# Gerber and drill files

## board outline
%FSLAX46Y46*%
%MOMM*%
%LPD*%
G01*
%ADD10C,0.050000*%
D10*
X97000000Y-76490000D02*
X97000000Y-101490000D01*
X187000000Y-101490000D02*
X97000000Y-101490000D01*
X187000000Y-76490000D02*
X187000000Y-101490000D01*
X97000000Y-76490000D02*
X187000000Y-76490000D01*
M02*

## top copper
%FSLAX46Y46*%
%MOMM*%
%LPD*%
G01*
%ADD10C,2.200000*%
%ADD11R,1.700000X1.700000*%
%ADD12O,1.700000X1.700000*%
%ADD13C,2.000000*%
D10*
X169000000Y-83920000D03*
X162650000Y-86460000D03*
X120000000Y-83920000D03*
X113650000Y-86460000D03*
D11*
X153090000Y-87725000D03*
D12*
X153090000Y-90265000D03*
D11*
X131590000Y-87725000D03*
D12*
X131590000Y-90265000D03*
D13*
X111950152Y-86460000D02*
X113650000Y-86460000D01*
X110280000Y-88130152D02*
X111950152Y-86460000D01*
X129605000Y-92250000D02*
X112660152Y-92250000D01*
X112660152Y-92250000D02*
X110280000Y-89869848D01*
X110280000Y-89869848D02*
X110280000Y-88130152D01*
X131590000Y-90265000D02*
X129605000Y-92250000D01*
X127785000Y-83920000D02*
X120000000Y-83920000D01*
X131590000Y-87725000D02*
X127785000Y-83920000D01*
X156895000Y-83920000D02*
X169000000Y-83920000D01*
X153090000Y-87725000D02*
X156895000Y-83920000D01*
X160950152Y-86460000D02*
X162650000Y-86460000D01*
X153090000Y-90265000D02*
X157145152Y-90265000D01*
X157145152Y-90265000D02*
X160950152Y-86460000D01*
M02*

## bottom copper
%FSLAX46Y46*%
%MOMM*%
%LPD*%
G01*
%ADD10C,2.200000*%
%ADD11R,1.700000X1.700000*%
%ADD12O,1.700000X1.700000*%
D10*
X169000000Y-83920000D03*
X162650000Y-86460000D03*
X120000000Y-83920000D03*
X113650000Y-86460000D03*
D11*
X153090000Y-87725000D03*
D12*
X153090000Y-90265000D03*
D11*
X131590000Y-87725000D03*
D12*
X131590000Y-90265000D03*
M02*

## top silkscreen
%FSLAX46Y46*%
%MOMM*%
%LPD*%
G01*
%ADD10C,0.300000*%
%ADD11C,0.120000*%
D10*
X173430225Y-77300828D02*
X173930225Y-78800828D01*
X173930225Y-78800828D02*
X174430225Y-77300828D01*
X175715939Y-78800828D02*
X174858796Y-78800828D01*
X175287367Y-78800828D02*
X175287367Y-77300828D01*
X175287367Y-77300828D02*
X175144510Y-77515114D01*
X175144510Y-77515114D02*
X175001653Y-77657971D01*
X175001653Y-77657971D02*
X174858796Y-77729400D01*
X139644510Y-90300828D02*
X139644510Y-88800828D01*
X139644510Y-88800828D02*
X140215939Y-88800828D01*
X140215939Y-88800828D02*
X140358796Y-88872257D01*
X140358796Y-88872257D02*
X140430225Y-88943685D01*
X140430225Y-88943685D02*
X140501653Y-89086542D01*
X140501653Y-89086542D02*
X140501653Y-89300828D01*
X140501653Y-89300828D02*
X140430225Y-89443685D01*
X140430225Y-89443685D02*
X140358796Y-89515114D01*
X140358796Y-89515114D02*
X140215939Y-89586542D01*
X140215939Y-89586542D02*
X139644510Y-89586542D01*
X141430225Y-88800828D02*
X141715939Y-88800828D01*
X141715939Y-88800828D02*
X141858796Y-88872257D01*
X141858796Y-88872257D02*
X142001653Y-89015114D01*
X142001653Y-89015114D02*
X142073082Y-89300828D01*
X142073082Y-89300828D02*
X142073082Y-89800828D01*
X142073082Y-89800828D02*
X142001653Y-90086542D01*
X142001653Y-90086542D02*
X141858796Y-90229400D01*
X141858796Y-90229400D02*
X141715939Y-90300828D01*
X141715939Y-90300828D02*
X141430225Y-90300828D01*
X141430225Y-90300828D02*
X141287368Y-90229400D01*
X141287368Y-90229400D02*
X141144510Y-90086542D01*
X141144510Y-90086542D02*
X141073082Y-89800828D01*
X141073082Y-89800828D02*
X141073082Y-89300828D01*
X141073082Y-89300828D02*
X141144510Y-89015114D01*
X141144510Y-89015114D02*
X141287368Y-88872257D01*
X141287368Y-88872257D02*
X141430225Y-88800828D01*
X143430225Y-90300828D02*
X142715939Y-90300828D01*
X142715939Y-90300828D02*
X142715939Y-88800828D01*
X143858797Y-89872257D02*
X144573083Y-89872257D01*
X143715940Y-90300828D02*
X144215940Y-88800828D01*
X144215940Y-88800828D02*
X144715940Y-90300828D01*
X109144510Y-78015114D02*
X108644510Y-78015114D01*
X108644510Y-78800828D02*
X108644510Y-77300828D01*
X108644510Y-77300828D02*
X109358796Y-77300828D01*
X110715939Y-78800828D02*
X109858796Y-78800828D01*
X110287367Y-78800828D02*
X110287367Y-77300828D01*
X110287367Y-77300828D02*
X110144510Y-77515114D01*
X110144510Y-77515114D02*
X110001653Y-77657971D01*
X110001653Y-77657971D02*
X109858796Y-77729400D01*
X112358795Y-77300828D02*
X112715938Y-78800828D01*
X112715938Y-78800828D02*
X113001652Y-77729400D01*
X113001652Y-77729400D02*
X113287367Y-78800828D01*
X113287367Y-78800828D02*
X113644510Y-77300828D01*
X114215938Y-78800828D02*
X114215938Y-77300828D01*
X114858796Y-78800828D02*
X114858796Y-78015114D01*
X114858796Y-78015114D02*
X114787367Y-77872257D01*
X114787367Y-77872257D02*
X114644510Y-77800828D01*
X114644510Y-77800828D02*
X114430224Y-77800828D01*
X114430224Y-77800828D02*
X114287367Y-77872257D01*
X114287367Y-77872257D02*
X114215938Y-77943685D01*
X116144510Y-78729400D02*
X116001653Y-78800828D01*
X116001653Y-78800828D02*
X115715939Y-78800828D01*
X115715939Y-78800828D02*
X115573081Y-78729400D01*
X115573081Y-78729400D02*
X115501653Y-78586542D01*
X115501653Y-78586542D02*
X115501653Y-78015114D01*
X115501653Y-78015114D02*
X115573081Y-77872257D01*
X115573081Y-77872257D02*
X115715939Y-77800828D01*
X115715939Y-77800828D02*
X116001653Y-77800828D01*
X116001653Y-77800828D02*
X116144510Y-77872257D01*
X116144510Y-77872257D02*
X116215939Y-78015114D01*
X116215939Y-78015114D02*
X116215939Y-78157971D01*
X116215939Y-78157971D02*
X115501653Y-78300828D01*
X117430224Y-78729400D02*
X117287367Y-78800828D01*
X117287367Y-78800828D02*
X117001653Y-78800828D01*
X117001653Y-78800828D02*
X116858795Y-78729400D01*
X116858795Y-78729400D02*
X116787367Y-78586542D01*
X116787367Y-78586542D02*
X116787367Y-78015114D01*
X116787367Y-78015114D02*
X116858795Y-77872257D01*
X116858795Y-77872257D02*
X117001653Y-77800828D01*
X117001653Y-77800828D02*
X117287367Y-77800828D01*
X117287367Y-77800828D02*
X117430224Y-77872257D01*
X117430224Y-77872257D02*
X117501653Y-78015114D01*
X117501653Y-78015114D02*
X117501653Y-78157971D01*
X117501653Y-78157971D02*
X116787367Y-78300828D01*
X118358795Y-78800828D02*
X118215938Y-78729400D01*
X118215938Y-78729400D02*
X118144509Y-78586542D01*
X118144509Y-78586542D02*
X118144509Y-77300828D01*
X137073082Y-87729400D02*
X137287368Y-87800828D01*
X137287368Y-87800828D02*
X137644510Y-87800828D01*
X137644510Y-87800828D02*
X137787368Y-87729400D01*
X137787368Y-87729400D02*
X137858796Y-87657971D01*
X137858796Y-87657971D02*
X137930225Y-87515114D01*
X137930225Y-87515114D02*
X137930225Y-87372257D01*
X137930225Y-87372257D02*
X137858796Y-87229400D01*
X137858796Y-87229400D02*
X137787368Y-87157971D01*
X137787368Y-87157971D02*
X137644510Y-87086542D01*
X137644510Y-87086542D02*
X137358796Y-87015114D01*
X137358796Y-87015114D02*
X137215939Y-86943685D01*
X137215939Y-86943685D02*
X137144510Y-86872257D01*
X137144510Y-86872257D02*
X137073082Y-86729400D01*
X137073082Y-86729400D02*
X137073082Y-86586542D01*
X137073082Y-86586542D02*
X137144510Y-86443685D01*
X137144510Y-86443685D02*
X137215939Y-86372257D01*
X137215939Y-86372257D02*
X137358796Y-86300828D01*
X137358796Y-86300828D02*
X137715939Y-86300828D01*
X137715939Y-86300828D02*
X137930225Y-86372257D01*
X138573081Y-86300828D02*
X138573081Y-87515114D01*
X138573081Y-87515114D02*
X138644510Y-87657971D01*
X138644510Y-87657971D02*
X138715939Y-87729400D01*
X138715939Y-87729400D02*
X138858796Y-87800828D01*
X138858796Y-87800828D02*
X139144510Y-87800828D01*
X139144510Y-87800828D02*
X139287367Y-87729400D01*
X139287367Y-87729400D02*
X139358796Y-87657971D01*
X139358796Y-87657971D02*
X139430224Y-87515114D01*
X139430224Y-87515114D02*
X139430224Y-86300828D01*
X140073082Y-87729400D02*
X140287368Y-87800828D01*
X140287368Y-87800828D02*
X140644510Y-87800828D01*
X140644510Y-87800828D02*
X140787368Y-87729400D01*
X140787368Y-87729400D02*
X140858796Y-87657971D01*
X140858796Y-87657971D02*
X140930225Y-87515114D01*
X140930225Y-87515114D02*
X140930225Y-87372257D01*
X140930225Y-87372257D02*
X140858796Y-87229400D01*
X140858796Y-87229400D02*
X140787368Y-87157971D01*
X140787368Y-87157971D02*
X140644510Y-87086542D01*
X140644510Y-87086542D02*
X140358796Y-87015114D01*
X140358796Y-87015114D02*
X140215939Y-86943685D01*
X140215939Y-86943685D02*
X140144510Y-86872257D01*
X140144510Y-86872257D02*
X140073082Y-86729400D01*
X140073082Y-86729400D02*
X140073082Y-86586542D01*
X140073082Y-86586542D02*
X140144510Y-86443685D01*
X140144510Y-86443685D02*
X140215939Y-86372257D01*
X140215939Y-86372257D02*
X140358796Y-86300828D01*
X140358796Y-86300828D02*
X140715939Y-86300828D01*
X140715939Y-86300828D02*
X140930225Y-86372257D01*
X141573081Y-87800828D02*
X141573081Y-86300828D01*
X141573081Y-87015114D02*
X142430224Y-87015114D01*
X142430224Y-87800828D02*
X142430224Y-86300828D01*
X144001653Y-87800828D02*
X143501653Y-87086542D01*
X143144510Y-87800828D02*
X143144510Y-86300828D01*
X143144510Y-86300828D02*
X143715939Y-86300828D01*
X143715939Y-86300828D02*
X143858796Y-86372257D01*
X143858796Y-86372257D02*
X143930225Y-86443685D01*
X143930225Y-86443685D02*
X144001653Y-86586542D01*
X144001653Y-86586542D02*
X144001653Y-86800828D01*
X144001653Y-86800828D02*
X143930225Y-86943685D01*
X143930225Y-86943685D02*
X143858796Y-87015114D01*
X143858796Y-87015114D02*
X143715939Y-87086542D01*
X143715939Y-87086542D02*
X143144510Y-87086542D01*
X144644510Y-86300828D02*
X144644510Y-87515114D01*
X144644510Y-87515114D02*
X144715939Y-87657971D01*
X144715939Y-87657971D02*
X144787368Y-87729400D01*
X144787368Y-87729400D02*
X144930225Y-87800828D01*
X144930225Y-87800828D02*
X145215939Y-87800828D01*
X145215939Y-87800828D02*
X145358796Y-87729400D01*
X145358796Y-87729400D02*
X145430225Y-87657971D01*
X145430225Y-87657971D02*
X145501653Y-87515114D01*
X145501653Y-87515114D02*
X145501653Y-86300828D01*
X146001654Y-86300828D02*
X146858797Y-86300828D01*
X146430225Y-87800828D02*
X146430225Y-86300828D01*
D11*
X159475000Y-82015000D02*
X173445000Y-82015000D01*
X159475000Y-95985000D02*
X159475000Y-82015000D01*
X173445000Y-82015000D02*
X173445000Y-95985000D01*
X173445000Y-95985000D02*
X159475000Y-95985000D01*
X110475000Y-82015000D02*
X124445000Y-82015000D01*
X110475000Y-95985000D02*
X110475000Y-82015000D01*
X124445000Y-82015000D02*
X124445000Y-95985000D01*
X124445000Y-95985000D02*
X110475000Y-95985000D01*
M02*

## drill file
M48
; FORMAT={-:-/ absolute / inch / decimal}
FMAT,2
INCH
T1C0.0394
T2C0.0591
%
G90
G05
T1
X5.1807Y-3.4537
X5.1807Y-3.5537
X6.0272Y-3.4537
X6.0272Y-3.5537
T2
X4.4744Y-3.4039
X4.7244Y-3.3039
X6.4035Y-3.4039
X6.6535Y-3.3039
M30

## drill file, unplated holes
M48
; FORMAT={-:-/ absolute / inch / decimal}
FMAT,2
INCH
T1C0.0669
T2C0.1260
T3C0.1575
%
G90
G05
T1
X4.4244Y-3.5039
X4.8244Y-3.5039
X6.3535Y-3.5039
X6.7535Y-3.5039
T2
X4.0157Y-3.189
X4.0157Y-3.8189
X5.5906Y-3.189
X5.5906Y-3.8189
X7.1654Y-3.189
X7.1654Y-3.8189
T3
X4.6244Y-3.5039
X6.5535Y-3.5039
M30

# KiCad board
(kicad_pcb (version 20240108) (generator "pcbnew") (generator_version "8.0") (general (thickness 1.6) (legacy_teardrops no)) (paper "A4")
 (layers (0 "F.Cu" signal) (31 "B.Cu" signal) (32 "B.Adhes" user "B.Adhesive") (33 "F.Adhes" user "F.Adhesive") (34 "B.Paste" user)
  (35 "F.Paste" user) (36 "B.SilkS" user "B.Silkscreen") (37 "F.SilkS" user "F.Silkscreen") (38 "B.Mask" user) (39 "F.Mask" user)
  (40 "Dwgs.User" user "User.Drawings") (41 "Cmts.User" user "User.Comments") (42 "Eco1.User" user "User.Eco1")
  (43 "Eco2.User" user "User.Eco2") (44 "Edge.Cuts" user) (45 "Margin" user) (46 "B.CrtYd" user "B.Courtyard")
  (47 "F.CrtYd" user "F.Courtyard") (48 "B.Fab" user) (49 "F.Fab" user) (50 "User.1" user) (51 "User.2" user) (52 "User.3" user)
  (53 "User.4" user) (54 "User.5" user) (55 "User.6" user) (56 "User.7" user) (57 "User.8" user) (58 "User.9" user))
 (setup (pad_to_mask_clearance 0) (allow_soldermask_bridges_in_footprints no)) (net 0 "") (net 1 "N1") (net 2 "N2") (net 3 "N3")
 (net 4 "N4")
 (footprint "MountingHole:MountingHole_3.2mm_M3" (layer "F.Cu") (at 142 81)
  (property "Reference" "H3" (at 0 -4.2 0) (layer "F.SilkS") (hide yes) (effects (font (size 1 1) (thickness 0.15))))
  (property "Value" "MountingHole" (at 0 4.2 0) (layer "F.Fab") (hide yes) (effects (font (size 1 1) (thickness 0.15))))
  (pad "" np_thru_hole circle (at 0 0) (size 3.2 3.2) (drill 3.2) (layers "*.Cu" "*.Mask")))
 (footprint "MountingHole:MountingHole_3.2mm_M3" (layer "F.Cu") (at 142 97)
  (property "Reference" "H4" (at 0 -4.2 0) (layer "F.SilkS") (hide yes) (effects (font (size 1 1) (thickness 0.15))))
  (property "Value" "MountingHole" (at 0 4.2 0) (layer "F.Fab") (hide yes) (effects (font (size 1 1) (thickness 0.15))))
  (pad "" np_thru_hole circle (at 0 0) (size 3.2 3.2) (drill 3.2) (layers "*.Cu" "*.Mask")))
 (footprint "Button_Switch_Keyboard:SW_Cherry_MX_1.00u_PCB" (layer "F.Cu") (at 169 83.92)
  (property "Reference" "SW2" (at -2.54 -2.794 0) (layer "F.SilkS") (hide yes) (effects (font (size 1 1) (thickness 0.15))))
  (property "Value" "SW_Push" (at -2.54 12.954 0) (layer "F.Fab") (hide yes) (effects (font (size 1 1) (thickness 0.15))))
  (fp_line (start -9.525 -1.905) (end 4.445 -1.905) (stroke (width 0.12) (type solid)) (layer "F.SilkS"))
  (fp_line (start -9.525 12.065) (end -9.525 -1.905) (stroke (width 0.12) (type solid)) (layer "F.SilkS"))
  (fp_line (start 4.445 -1.905) (end 4.445 12.065) (stroke (width 0.12) (type solid)) (layer "F.SilkS"))
  (fp_line (start 4.445 12.065) (end -9.525 12.065) (stroke (width 0.12) (type solid)) (layer "F.SilkS"))
  (pad "" np_thru_hole circle (at -7.62 5.08) (size 1.7 1.7) (drill 1.7) (layers "*.Cu" "*.Mask"))
  (pad "" np_thru_hole circle (at -2.54 5.08) (size 4 4) (drill 4) (layers "*.Cu" "*.Mask"))
  (pad "" np_thru_hole circle (at 2.54 5.08) (size 1.7 1.7) (drill 1.7) (layers "*.Cu" "*.Mask"))
  (pad "1" thru_hole circle (at 0 0) (size 2.2 2.2) (drill 1.5) (layers "*.Cu" "*.Mask") (remove_unused_layers no) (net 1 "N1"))
  (pad "2" thru_hole circle (at -6.35 2.54) (size 2.2 2.2) (drill 1.5) (layers "*.Cu" "*.Mask") (remove_unused_layers no) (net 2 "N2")))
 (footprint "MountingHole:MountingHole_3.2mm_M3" (layer "F.Cu") (at 182 97)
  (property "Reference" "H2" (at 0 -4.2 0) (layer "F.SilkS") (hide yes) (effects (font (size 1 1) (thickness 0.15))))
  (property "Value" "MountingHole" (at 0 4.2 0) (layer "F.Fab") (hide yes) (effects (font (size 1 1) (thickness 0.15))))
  (pad "" np_thru_hole circle (at 0 0) (size 3.2 3.2) (drill 3.2) (layers "*.Cu" "*.Mask")))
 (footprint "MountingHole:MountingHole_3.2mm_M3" (layer "F.Cu") (at 102 97)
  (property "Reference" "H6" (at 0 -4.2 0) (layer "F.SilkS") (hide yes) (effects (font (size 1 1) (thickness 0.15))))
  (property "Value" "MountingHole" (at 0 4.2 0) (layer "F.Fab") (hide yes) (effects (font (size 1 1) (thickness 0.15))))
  (pad "" np_thru_hole circle (at 0 0) (size 3.2 3.2) (drill 3.2) (layers "*.Cu" "*.Mask")))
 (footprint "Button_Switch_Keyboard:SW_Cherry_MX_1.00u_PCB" (layer "F.Cu") (at 120 83.92)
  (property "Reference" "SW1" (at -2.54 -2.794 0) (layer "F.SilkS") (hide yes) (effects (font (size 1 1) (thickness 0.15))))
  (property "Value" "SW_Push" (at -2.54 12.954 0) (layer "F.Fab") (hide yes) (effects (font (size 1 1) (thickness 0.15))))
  (fp_line (start -9.525 -1.905) (end 4.445 -1.905) (stroke (width 0.12) (type solid)) (layer "F.SilkS"))
  (fp_line (start -9.525 12.065) (end -9.525 -1.905) (stroke (width 0.12) (type solid)) (layer "F.SilkS"))
  (fp_line (start 4.445 -1.905) (end 4.445 12.065) (stroke (width 0.12) (type solid)) (layer "F.SilkS"))
  (fp_line (start 4.445 12.065) (end -9.525 12.065) (stroke (width 0.12) (type solid)) (layer "F.SilkS"))
  (pad "" np_thru_hole circle (at -7.62 5.08) (size 1.7 1.7) (drill 1.7) (layers "*.Cu" "*.Mask"))
  (pad "" np_thru_hole circle (at -2.54 5.08) (size 4 4) (drill 4) (layers "*.Cu" "*.Mask"))
  (pad "" np_thru_hole circle (at 2.54 5.08) (size 1.7 1.7) (drill 1.7) (layers "*.Cu" "*.Mask"))
  (pad "1" thru_hole circle (at 0 0) (size 2.2 2.2) (drill 1.5) (layers "*.Cu" "*.Mask") (remove_unused_layers no) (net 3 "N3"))
  (pad "2" thru_hole circle (at -6.35 2.54) (size 2.2 2.2) (drill 1.5) (layers "*.Cu" "*.Mask") (remove_unused_layers no) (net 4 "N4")))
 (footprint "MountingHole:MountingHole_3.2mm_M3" (layer "F.Cu") (at 182 81)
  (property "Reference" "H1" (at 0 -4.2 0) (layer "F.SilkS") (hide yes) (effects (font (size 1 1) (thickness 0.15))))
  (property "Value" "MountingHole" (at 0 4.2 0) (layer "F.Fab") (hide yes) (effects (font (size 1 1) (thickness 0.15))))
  (pad "" np_thru_hole circle (at 0 0) (size 3.2 3.2) (drill 3.2) (layers "*.Cu" "*.Mask")))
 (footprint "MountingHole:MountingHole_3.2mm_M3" (layer "F.Cu") (at 102 81)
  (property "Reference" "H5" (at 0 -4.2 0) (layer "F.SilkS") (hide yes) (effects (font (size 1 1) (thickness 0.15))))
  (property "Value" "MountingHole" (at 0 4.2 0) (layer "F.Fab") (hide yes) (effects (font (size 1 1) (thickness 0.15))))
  (pad "" np_thru_hole circle (at 0 0) (size 3.2 3.2) (drill 3.2) (layers "*.Cu" "*.Mask")))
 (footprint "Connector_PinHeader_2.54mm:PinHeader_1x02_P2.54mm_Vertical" (layer "B.Cu") (at 153.09 87.725 180)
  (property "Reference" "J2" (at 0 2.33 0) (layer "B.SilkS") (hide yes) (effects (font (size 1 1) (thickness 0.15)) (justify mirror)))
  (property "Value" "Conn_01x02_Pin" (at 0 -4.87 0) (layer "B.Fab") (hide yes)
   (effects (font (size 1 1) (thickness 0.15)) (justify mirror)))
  (pad "1" thru_hole rect (at 0 0 180) (size 1.7 1.7) (drill 1) (layers "*.Cu" "*.Mask") (remove_unused_layers no) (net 1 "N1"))
  (pad "2" thru_hole oval (at 0 -2.54 180) (size 1.7 1.7) (drill 1) (layers "*.Cu" "*.Mask") (remove_unused_layers no) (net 2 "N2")))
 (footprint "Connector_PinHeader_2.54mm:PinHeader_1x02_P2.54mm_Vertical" (layer "B.Cu") (at 131.59 87.725 180)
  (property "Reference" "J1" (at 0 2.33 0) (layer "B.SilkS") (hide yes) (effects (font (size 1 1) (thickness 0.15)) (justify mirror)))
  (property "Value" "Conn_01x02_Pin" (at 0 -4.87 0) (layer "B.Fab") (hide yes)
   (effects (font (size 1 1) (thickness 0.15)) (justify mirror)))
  (pad "1" thru_hole rect (at 0 0 180) (size 1.7 1.7) (drill 1) (layers "*.Cu" "*.Mask") (remove_unused_layers no) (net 3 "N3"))
  (pad "2" thru_hole oval (at 0 -2.54 180) (size 1.7 1.7) (drill 1) (layers "*.Cu" "*.Mask") (remove_unused_layers no) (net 4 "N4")))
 (gr_line (start 97 76.49) (end 97 101.49) (stroke (width 0.05) (type default)) (layer "Edge.Cuts"))
 (gr_line (start 187 101.49) (end 97 101.49) (stroke (width 0.05) (type default)) (layer "Edge.Cuts"))
 (gr_line (start 187 76.49) (end 187 101.49) (stroke (width 0.05) (type default)) (layer "Edge.Cuts"))
 (gr_line (start 97 76.49) (end 187 76.49) (stroke (width 0.05) (type default)) (layer "Edge.Cuts"))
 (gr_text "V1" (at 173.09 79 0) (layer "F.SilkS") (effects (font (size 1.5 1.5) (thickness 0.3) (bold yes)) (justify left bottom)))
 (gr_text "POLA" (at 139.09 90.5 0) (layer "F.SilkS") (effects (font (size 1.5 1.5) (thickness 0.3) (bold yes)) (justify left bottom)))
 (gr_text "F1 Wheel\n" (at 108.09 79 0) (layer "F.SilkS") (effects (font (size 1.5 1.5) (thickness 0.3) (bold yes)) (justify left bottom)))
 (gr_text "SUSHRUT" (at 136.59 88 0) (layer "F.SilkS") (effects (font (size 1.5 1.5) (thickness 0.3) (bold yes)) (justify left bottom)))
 (segment (start 111.950152 86.46) (end 113.65 86.46) (width 2) (layer "F.Cu") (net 4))
 (segment (start 110.28 88.130152) (end 111.950152 86.46) (width 2) (layer "F.Cu") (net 4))
 (segment (start 129.605 92.25) (end 112.660152 92.25) (width 2) (layer "F.Cu") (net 4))
 (segment (start 112.660152 92.25) (end 110.28 89.869848) (width 2) (layer "F.Cu") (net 4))
 (segment (start 110.28 89.869848) (end 110.28 88.130152) (width 2) (layer "F.Cu") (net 4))
 (segment (start 131.59 90.265) (end 129.605 92.25) (width 2) (layer "F.Cu") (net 4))
 (segment (start 127.785 83.92) (end 120 83.92) (width 2) (layer "F.Cu") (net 3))
 (segment (start 131.59 87.725) (end 127.785 83.92) (width 2) (layer "F.Cu") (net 3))
 (segment (start 156.895 83.92) (end 169 83.92) (width 2) (layer "F.Cu") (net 1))
 (segment (start 153.09 87.725) (end 156.895 83.92) (width 2) (layer "F.Cu") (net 1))
 (segment (start 160.950152 86.46) (end 162.65 86.46) (width 2) (layer "F.Cu") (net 2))
 (segment (start 153.09 90.265) (end 157.145152 90.265) (width 2) (layer "F.Cu") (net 2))
 (segment (start 157.145152 90.265) (end 160.950152 86.46) (width 2) (layer "F.Cu") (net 2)))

